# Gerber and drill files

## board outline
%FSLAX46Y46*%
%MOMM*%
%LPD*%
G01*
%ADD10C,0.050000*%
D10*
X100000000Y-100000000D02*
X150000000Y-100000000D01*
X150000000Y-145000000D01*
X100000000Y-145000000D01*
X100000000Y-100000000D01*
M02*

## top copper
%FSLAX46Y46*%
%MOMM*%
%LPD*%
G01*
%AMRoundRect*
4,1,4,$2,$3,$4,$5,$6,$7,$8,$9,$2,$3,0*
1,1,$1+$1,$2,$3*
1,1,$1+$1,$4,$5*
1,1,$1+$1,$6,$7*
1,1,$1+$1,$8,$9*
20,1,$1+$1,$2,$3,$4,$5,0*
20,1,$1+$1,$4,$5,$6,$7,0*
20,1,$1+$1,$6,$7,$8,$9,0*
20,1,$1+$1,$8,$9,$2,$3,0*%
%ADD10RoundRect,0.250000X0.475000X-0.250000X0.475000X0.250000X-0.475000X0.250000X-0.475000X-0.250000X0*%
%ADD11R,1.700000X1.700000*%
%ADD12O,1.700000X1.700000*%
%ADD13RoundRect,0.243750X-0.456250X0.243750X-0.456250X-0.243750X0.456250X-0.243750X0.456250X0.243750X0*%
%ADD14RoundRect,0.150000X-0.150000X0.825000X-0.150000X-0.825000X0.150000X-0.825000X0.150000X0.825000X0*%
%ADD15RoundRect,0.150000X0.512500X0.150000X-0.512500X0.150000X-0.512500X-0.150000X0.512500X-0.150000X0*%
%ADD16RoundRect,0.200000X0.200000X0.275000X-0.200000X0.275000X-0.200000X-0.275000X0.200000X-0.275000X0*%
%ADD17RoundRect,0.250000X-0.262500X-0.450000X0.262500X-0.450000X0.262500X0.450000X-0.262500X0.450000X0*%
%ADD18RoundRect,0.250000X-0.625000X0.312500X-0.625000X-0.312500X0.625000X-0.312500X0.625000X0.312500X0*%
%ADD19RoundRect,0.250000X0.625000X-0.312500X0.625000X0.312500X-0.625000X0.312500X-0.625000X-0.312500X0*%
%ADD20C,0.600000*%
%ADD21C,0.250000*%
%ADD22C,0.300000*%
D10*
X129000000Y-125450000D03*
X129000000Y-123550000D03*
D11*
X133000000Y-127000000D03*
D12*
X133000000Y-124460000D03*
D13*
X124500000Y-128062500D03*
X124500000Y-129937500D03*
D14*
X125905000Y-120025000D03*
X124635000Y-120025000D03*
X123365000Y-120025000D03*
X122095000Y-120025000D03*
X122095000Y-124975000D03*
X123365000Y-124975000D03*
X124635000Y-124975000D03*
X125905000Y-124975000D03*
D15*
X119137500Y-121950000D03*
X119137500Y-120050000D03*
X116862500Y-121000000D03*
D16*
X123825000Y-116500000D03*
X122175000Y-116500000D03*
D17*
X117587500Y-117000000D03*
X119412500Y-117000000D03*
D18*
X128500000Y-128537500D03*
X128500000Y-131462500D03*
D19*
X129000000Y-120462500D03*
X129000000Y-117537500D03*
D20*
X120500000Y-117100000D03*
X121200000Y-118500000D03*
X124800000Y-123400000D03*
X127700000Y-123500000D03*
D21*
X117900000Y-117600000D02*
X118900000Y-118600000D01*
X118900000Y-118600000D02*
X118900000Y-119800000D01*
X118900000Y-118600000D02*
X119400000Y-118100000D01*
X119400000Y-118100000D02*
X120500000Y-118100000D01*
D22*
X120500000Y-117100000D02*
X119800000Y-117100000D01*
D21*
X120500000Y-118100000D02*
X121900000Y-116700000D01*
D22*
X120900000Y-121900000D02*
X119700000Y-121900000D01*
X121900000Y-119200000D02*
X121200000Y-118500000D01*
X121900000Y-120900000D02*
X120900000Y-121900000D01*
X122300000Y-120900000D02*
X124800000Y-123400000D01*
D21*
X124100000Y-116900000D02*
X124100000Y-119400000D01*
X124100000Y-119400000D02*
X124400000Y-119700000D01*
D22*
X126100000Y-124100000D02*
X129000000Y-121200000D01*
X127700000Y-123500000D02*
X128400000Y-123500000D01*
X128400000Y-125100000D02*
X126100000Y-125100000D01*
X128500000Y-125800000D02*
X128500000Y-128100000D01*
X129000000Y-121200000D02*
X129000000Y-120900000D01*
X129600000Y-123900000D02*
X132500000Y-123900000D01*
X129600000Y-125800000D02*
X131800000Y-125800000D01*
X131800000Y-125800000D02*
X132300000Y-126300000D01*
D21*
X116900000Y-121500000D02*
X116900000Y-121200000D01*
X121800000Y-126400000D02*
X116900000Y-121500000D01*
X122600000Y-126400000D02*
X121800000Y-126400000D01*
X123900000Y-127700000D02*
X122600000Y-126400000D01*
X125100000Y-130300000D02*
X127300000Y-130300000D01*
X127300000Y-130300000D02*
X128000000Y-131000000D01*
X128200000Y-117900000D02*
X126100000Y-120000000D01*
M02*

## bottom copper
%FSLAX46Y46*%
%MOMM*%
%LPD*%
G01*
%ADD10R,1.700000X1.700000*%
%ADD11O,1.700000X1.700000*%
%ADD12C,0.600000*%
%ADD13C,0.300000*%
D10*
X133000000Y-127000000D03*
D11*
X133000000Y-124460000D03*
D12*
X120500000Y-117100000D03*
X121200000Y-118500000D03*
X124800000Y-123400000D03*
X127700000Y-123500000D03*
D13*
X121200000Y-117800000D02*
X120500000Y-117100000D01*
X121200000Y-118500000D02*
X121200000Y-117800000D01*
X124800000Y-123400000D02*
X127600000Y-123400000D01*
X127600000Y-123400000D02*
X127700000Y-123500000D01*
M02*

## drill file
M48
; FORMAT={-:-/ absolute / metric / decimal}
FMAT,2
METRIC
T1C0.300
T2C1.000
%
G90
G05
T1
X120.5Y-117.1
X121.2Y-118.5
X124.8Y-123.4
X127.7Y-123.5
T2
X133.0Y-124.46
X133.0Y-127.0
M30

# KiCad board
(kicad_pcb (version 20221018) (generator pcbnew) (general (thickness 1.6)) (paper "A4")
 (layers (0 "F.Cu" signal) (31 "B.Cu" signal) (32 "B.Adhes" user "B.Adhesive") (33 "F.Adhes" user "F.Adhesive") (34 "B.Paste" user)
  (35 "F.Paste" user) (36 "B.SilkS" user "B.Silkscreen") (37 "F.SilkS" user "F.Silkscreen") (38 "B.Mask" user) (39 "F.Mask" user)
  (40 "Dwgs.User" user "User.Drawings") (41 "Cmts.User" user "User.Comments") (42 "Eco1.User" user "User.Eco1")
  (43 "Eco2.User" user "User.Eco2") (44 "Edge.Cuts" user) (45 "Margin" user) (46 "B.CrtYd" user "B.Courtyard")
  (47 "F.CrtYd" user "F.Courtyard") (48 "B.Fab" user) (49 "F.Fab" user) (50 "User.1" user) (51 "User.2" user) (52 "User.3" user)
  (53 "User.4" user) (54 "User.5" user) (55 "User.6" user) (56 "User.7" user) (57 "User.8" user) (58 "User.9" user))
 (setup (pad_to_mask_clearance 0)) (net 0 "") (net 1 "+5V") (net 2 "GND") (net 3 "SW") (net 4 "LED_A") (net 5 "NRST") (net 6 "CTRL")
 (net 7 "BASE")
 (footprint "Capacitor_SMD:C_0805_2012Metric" (layer "F.Cu") (at 129 124.5 90)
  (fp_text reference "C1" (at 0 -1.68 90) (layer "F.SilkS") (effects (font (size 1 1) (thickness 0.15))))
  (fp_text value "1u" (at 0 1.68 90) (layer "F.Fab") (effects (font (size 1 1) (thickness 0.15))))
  (pad "1" smd roundrect (at -0.95 0 90) (size 1 1.45) (layers "F.Cu" "F.Paste" "F.Mask") (roundrect_rratio 0.25) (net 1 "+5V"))
  (pad "2" smd roundrect (at 0.95 0 90) (size 1 1.45) (layers "F.Cu" "F.Paste" "F.Mask") (roundrect_rratio 0.25) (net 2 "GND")))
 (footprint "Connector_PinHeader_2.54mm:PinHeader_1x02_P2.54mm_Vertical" (layer "F.Cu") (at 133 127 180)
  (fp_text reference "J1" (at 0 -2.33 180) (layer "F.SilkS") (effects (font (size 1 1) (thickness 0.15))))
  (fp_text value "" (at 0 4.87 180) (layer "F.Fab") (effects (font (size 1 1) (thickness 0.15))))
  (pad "1" thru_hole rect (at 0 0 180) (size 1.7 1.7) (drill 1) (layers "*.Cu" "*.Mask") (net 1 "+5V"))
  (pad "2" thru_hole oval (at 0 2.54 180) (size 1.7 1.7) (drill 1) (layers "*.Cu" "*.Mask") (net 2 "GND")))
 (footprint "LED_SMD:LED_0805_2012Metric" (layer "F.Cu") (at 124.5 129 -90)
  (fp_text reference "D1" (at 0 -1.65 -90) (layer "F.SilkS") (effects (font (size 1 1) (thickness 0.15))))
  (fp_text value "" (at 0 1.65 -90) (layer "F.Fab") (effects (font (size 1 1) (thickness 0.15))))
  (pad "1" smd roundrect (at -0.9375 0 270) (size 0.975 1.4) (layers "F.Cu" "F.Paste" "F.Mask") (roundrect_rratio 0.25) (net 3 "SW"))
  (pad "2" smd roundrect (at 0.9375 0 270) (size 0.975 1.4) (layers "F.Cu" "F.Paste" "F.Mask") (roundrect_rratio 0.25) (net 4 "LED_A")))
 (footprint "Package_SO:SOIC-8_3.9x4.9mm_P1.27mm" (layer "F.Cu") (at 124 122.5 -90)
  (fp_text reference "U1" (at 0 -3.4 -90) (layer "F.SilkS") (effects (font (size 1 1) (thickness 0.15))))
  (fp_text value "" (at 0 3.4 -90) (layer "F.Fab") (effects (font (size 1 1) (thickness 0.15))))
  (pad "1" smd roundrect (at -2.475 -1.905 270) (size 1.95 0.6) (layers "F.Cu" "F.Paste" "F.Mask") (roundrect_rratio 0.25) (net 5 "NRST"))
  (pad "2" smd roundrect (at -2.475 -0.635 270) (size 1.95 0.6) (layers "F.Cu" "F.Paste" "F.Mask") (roundrect_rratio 0.25) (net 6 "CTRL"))
  (pad "3" smd roundrect (at -2.475 0.635 270) (size 1.95 0.6) (layers "F.Cu" "F.Paste" "F.Mask") (roundrect_rratio 0.25))
  (pad "4" smd roundrect (at -2.475 1.905 270) (size 1.95 0.6) (layers "F.Cu" "F.Paste" "F.Mask") (roundrect_rratio 0.25) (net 2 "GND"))
  (pad "5" smd roundrect (at 2.475 1.905 270) (size 1.95 0.6) (layers "F.Cu" "F.Paste" "F.Mask") (roundrect_rratio 0.25))
  (pad "6" smd roundrect (at 2.475 0.635 270) (size 1.95 0.6) (layers "F.Cu" "F.Paste" "F.Mask") (roundrect_rratio 0.25))
  (pad "7" smd roundrect (at 2.475 -0.635 270) (size 1.95 0.6) (layers "F.Cu" "F.Paste" "F.Mask") (roundrect_rratio 0.25))
  (pad "8" smd roundrect (at 2.475 -1.905 270) (size 1.95 0.6) (layers "F.Cu" "F.Paste" "F.Mask") (roundrect_rratio 0.25) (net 1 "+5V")))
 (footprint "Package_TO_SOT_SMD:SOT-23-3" (layer "F.Cu") (at 118 121 180)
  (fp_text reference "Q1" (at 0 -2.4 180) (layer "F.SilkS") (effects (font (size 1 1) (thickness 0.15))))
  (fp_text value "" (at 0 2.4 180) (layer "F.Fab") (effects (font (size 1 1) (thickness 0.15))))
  (pad "1" smd roundrect (at -1.1375 -0.95 180) (size 1.325 0.6) (layers "F.Cu" "F.Paste" "F.Mask") (roundrect_rratio 0.25) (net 2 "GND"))
  (pad "2" smd roundrect (at -1.1375 0.95 180) (size 1.325 0.6) (layers "F.Cu" "F.Paste" "F.Mask") (roundrect_rratio 0.25) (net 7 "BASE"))
  (pad "3" smd roundrect (at 1.1375 0 180) (size 1.325 0.6) (layers "F.Cu" "F.Paste" "F.Mask") (roundrect_rratio 0.25) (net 3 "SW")))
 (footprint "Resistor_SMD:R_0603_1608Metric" (layer "F.Cu") (at 123 116.5 180)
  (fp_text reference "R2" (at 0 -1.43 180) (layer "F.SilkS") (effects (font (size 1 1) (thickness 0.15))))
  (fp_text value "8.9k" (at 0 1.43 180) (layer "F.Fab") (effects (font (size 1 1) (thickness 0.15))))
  (pad "1" smd roundrect (at -0.825 0 180) (size 0.8 0.95) (layers "F.Cu" "F.Paste" "F.Mask") (roundrect_rratio 0.25) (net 6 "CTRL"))
  (pad "2" smd roundrect (at 0.825 0 180) (size 0.8 0.95) (layers "F.Cu" "F.Paste" "F.Mask") (roundrect_rratio 0.25) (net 7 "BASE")))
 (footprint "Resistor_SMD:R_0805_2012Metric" (layer "F.Cu") (at 118.5 117)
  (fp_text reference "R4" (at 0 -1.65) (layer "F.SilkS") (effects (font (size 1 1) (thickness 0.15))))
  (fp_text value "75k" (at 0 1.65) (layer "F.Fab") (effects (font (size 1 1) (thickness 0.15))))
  (pad "1" smd roundrect (at -0.9125 0) (size 1.025 1.4) (layers "F.Cu" "F.Paste" "F.Mask") (roundrect_rratio 0.243902) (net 7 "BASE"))
  (pad "2" smd roundrect (at 0.9125 0) (size 1.025 1.4) (layers "F.Cu" "F.Paste" "F.Mask") (roundrect_rratio 0.243902) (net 2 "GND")))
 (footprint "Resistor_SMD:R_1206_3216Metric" (layer "F.Cu") (at 128.5 130 -90)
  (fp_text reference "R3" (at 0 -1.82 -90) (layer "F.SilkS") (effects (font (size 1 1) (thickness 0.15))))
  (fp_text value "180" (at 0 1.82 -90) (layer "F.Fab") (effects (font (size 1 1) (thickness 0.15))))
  (pad "1" smd roundrect (at -1.4625 0 270) (size 1.125 1.75) (layers "F.Cu" "F.Paste" "F.Mask") (roundrect_rratio 0.222222) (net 1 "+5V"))
  (pad "2" smd roundrect (at 1.4625 0 270) (size 1.125 1.75) (layers "F.Cu" "F.Paste" "F.Mask") (roundrect_rratio 0.222222) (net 4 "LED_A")))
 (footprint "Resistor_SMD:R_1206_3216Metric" (layer "F.Cu") (at 129 119 90)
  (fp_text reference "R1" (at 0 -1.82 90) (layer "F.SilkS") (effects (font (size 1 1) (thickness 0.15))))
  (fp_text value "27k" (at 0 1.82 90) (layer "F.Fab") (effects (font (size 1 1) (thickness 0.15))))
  (pad "1" smd roundrect (at -1.4625 0 90) (size 1.125 1.75) (layers "F.Cu" "F.Paste" "F.Mask") (roundrect_rratio 0.222222) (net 1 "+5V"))
  (pad "2" smd roundrect (at 1.4625 0 90) (size 1.125 1.75) (layers "F.Cu" "F.Paste" "F.Mask") (roundrect_rratio 0.222222) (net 5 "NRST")))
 (gr_rect (start 100 100) (end 150 145) (stroke (width 0.05) (type default)) (fill none) (layer "Edge.Cuts"))
 (segment (start 117.9 117.6) (end 118.9 118.6) (width 0.25) (layer "F.Cu") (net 7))
 (segment (start 118.9 118.6) (end 118.9 119.8) (width 0.25) (layer "F.Cu") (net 7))
 (segment (start 118.9 118.6) (end 119.4 118.1) (width 0.25) (layer "F.Cu") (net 7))
 (segment (start 119.4 118.1) (end 120.5 118.1) (width 0.25) (layer "F.Cu") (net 7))
 (segment (start 120.5 117.1) (end 119.8 117.1) (width 0.3) (layer "F.Cu") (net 2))
 (segment (start 120.5 118.1) (end 121.9 116.7) (width 0.25) (layer "F.Cu") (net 7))
 (segment (start 120.9 121.9) (end 119.7 121.9) (width 0.3) (layer "F.Cu") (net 2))
 (segment (start 121.9 119.2) (end 121.2 118.5) (width 0.3) (layer "F.Cu") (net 2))
 (segment (start 121.9 120.9) (end 120.9 121.9) (width 0.3) (layer "F.Cu") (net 2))
 (segment (start 122.3 120.9) (end 124.8 123.4) (width 0.3) (layer "F.Cu") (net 2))
 (segment (start 124.1 116.9) (end 124.1 119.4) (width 0.25) (layer "F.Cu") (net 6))
 (segment (start 124.1 119.4) (end 124.4 119.7) (width 0.25) (layer "F.Cu") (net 6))
 (segment (start 126.1 124.1) (end 129 121.2) (width 0.3) (layer "F.Cu") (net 1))
 (segment (start 127.7 123.5) (end 128.4 123.5) (width 0.3) (layer "F.Cu") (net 2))
 (segment (start 128.4 125.1) (end 126.1 125.1) (width 0.3) (layer "F.Cu") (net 1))
 (segment (start 128.5 125.8) (end 128.5 128.1) (width 0.3) (layer "F.Cu") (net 1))
 (segment (start 129 121.2) (end 129 120.9) (width 0.3) (layer "F.Cu") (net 1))
 (segment (start 129.6 123.9) (end 132.5 123.9) (width 0.3) (layer "F.Cu") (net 2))
 (segment (start 129.6 125.8) (end 131.8 125.8) (width 0.3) (layer "F.Cu") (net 1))
 (segment (start 131.8 125.8) (end 132.3 126.3) (width 0.3) (layer "F.Cu") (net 1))
 (via (at 120.5 117.1) (size 0.6) (drill 0.3) (layers "F.Cu" "B.Cu") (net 2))
 (via (at 121.2 118.5) (size 0.6) (drill 0.3) (layers "F.Cu" "B.Cu") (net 2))
 (via (at 124.8 123.4) (size 0.6) (drill 0.3) (layers "F.Cu" "B.Cu") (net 2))
 (via (at 127.7 123.5) (size 0.6) (drill 0.3) (layers "F.Cu" "B.Cu") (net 2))
 (segment (start 116.9 121.5) (end 116.9 121.2) (width 0.25) (layer "F.Cu") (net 3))
 (segment (start 121.2 117.8) (end 120.5 117.1) (width 0.3) (layer "B.Cu") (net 2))
 (segment (start 121.2 118.5) (end 121.2 117.8) (width 0.3) (layer "B.Cu") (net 2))
 (segment (start 121.8 126.4) (end 116.9 121.5) (width 0.25) (layer "F.Cu") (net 3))
 (segment (start 122.6 126.4) (end 121.8 126.4) (width 0.25) (layer "F.Cu") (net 3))
 (segment (start 123.9 127.7) (end 122.6 126.4) (width 0.25) (layer "F.Cu") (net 3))
 (segment (start 124.8 123.4) (end 127.6 123.4) (width 0.3) (layer "B.Cu") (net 2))
 (segment (start 125.1 130.3) (end 127.3 130.3) (width 0.25) (layer "F.Cu") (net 4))
 (segment (start 127.3 130.3) (end 128 131) (width 0.25) (layer "F.Cu") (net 4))
 (segment (start 127.6 123.4) (end 127.7 123.5) (width 0.3) (layer "B.Cu") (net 2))
 (segment (start 128.2 117.9) (end 126.1 120) (width 0.25) (layer "F.Cu") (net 5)))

